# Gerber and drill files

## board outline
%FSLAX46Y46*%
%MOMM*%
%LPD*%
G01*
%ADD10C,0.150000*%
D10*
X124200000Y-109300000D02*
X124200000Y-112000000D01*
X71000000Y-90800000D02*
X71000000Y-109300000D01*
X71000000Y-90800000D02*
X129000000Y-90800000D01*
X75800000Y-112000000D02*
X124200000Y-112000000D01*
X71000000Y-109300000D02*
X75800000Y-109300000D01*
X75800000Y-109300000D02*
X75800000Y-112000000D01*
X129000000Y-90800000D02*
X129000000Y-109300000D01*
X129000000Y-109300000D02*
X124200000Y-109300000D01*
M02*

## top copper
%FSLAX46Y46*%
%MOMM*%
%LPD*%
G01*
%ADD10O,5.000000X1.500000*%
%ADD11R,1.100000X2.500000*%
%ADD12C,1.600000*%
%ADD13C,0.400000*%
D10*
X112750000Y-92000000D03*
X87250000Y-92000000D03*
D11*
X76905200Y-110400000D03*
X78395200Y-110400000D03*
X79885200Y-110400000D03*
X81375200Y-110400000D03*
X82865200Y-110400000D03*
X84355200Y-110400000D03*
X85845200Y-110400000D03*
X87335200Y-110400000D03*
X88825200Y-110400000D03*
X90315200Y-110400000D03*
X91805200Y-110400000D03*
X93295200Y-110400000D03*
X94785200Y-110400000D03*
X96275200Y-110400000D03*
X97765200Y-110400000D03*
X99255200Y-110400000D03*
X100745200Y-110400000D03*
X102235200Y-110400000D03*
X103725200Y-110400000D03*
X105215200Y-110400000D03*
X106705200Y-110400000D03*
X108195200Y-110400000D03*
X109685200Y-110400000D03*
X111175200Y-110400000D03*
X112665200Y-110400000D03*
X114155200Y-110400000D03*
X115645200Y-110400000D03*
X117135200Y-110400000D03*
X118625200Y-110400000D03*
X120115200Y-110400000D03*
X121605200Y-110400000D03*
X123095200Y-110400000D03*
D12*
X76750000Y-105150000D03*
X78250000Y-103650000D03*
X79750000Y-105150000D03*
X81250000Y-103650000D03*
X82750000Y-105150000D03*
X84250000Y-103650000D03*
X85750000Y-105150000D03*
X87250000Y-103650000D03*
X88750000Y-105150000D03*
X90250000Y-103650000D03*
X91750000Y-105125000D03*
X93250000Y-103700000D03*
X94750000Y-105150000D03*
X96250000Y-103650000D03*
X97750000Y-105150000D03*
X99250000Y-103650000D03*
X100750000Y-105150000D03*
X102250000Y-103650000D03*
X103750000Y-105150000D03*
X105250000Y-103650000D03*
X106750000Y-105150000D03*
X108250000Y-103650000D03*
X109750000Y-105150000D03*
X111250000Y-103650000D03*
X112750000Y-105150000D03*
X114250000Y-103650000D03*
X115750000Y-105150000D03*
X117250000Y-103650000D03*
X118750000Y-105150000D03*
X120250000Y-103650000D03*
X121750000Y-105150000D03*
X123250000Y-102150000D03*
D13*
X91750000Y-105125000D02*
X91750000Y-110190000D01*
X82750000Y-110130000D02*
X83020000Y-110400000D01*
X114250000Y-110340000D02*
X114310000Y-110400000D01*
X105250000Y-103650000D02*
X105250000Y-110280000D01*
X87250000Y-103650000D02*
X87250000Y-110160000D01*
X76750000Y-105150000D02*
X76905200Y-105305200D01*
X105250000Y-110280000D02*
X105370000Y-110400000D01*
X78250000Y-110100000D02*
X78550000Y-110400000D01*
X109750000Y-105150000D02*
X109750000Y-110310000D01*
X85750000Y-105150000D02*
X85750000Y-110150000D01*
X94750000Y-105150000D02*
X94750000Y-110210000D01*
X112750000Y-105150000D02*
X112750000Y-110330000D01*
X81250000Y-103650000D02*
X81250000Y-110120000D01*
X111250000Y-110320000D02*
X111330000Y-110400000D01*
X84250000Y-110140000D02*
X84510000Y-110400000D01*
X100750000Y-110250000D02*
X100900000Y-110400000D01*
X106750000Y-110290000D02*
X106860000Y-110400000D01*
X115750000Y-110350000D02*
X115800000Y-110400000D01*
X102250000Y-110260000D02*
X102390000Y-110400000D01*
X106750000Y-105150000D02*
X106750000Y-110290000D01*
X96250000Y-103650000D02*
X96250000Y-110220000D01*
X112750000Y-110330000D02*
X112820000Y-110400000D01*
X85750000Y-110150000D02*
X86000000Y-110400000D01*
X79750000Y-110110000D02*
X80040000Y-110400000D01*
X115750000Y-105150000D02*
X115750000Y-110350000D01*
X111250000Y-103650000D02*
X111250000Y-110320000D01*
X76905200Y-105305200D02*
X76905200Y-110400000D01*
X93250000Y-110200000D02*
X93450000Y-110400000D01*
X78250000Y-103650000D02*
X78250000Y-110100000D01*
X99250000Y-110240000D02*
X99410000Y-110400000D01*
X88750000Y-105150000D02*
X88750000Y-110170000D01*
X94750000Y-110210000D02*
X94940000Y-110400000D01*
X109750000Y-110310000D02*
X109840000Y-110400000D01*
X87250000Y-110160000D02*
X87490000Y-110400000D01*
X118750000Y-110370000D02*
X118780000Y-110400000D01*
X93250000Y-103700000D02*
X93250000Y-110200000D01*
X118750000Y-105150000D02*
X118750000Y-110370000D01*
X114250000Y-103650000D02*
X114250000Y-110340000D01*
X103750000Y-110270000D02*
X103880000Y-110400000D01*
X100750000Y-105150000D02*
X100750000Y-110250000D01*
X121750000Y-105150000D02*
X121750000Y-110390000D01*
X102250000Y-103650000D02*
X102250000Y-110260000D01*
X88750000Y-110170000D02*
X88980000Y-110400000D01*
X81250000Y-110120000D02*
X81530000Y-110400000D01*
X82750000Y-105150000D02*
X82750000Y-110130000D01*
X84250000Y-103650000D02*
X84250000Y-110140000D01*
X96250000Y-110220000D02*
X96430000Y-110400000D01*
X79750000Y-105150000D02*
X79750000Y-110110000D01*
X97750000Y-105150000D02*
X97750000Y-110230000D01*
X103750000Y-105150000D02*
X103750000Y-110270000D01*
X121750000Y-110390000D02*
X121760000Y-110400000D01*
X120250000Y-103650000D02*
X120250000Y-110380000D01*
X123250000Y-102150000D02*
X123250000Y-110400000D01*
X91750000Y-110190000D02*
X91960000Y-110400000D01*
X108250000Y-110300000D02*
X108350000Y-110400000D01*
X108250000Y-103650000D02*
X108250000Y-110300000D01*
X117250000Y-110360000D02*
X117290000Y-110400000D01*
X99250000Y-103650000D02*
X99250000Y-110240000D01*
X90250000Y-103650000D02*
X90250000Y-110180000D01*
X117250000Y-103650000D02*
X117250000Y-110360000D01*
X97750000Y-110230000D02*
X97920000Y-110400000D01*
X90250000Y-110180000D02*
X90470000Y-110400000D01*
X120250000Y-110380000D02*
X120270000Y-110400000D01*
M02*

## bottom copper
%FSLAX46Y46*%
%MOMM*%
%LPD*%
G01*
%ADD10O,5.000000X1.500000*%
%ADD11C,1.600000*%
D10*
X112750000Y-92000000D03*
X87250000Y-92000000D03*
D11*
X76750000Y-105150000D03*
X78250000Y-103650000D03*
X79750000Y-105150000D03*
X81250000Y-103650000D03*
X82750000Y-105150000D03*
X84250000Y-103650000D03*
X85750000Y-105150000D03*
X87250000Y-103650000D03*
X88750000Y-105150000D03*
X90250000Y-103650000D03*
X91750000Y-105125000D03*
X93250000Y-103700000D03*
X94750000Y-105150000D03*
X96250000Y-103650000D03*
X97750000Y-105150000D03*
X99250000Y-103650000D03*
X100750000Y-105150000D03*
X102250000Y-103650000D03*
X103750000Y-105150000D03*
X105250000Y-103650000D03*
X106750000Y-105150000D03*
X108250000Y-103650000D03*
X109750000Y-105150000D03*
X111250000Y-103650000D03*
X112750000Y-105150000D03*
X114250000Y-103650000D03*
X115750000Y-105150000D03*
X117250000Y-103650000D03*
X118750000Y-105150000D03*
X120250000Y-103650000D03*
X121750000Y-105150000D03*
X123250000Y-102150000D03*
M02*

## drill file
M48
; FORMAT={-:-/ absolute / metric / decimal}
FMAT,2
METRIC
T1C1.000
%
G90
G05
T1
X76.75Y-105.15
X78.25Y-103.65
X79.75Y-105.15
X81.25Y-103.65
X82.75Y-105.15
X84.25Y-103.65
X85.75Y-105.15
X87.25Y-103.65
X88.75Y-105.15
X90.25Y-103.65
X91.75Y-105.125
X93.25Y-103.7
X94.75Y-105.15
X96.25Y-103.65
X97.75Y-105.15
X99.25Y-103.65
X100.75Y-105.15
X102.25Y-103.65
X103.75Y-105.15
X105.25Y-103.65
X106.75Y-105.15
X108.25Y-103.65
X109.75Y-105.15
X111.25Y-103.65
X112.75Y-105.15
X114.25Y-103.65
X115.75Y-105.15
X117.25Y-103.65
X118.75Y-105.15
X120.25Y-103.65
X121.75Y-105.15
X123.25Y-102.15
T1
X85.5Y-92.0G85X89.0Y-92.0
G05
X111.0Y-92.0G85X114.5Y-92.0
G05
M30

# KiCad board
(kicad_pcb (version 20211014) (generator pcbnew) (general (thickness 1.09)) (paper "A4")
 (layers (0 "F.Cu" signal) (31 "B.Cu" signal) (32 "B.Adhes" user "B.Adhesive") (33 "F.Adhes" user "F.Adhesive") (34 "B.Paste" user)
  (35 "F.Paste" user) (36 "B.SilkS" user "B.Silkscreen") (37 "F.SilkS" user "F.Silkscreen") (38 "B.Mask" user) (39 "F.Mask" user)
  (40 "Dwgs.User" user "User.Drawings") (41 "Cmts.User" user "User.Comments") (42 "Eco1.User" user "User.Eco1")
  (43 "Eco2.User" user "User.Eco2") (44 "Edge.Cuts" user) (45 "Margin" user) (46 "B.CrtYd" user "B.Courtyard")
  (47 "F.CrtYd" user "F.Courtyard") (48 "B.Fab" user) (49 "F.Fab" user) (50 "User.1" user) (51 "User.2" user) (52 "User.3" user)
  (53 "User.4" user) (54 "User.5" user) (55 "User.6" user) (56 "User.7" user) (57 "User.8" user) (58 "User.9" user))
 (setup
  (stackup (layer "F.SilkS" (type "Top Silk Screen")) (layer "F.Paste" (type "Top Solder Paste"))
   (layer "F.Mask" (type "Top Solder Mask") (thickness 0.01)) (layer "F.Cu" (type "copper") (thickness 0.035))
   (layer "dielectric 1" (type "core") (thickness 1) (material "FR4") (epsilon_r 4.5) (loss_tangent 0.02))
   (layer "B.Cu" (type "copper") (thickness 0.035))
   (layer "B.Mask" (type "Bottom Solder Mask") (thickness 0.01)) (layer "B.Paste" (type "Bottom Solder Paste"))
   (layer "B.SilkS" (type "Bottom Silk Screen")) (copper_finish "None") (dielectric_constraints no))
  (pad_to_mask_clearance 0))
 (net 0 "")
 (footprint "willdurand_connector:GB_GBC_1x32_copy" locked (layer "F.Cu") (at 100 100)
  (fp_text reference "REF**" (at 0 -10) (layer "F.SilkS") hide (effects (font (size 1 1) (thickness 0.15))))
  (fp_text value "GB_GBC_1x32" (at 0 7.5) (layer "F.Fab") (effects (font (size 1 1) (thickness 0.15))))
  (pad "" thru_hole oval locked (at 12.75 -8) (size 5 1.5) (drill oval 4.5 1) (layers *.Cu *.Mask))
  (pad "" thru_hole oval locked (at -12.75 -8) (size 5 1.5) (drill oval 4.5 1) (layers *.Cu *.Mask))
  (pad "1" connect rect locked (at -23.0948 10.4) (size 1.1 2.5) (layers "F.Cu" "F.Mask"))
  (pad "2" connect rect locked (at -21.6048 10.4) (size 1.1 2.5) (layers "F.Cu" "F.Mask"))
  (pad "3" connect rect locked (at -20.1148 10.4) (size 1.1 2.5) (layers "F.Cu" "F.Mask"))
  (pad "4" connect rect locked (at -18.6248 10.4) (size 1.1 2.5) (layers "F.Cu" "F.Mask"))
  (pad "5" connect rect locked (at -17.1348 10.4) (size 1.1 2.5) (layers "F.Cu" "F.Mask"))
  (pad "6" connect rect locked (at -15.6448 10.4) (size 1.1 2.5) (layers "F.Cu" "F.Mask"))
  (pad "7" connect rect locked (at -14.1548 10.4) (size 1.1 2.5) (layers "F.Cu" "F.Mask"))
  (pad "8" connect rect locked (at -12.6648 10.4) (size 1.1 2.5) (layers "F.Cu" "F.Mask"))
  (pad "9" connect rect locked (at -11.1748 10.4) (size 1.1 2.5) (layers "F.Cu" "F.Mask"))
  (pad "10" connect rect locked (at -9.6848 10.4) (size 1.1 2.5) (layers "F.Cu" "F.Mask"))
  (pad "11" connect rect locked (at -8.1948 10.4) (size 1.1 2.5) (layers "F.Cu" "F.Mask"))
  (pad "12" connect rect locked (at -6.7048 10.4) (size 1.1 2.5) (layers "F.Cu" "F.Mask"))
  (pad "13" connect rect locked (at -5.2148 10.4) (size 1.1 2.5) (layers "F.Cu" "F.Mask"))
  (pad "14" connect rect locked (at -3.7248 10.4) (size 1.1 2.5) (layers "F.Cu" "F.Mask"))
  (pad "15" connect rect locked (at -2.2348 10.4) (size 1.1 2.5) (layers "F.Cu" "F.Mask"))
  (pad "16" connect rect locked (at -0.7448 10.4) (size 1.1 2.5) (layers "F.Cu" "F.Mask"))
  (pad "17" connect rect locked (at 0.7452 10.4) (size 1.1 2.5) (layers "F.Cu" "F.Mask"))
  (pad "18" connect rect locked (at 2.2352 10.4) (size 1.1 2.5) (layers "F.Cu" "F.Mask"))
  (pad "19" connect rect locked (at 3.7252 10.4) (size 1.1 2.5) (layers "F.Cu" "F.Mask"))
  (pad "20" connect rect locked (at 5.2152 10.4) (size 1.1 2.5) (layers "F.Cu" "F.Mask"))
  (pad "21" connect rect locked (at 6.7052 10.4) (size 1.1 2.5) (layers "F.Cu" "F.Mask"))
  (pad "22" connect rect locked (at 8.1952 10.4) (size 1.1 2.5) (layers "F.Cu" "F.Mask"))
  (pad "23" connect rect locked (at 9.6852 10.4) (size 1.1 2.5) (layers "F.Cu" "F.Mask"))
  (pad "24" connect rect locked (at 11.1752 10.4) (size 1.1 2.5) (layers "F.Cu" "F.Mask"))
  (pad "25" connect rect locked (at 12.6652 10.4) (size 1.1 2.5) (layers "F.Cu" "F.Mask"))
  (pad "26" connect rect locked (at 14.1552 10.4) (size 1.1 2.5) (layers "F.Cu" "F.Mask"))
  (pad "27" connect rect locked (at 15.6452 10.4) (size 1.1 2.5) (layers "F.Cu" "F.Mask"))
  (pad "28" connect rect locked (at 17.1352 10.4) (size 1.1 2.5) (layers "F.Cu" "F.Mask"))
  (pad "29" connect rect locked (at 18.6252 10.4) (size 1.1 2.5) (layers "F.Cu" "F.Mask"))
  (pad "30" connect rect locked (at 20.1152 10.4) (size 1.1 2.5) (layers "F.Cu" "F.Mask"))
  (pad "31" connect rect locked (at 21.6052 10.4) (size 1.1 2.5) (layers "F.Cu" "F.Mask"))
  (pad "32" connect rect locked (at 23.0952 10.4) (size 1.1 2.5) (layers "F.Cu" "F.Mask")))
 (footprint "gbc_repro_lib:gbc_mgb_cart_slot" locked (layer "B.Cu") (at 100 105.15 180)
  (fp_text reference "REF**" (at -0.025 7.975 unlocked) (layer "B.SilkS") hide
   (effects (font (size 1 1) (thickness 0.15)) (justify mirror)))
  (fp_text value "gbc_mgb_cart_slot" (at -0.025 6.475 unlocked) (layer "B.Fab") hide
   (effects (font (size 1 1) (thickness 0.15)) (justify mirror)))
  (pad "1" thru_hole circle locked (at 23.25 0 180) (size 1.6 1.6) (drill 1) (layers *.Cu *.Mask))
  (pad "2" thru_hole circle locked (at 21.75 1.5 180) (size 1.6 1.6) (drill 1) (layers *.Cu *.Mask))
  (pad "3" thru_hole circle locked (at 20.25 0 180) (size 1.6 1.6) (drill 1) (layers *.Cu *.Mask))
  (pad "4" thru_hole circle locked (at 18.75 1.5 180) (size 1.6 1.6) (drill 1) (layers *.Cu *.Mask))
  (pad "5" thru_hole circle locked (at 17.25 0 180) (size 1.6 1.6) (drill 1) (layers *.Cu *.Mask))
  (pad "6" thru_hole circle locked (at 15.75 1.5 180) (size 1.6 1.6) (drill 1) (layers *.Cu *.Mask))
  (pad "7" thru_hole circle locked (at 14.25 0 180) (size 1.6 1.6) (drill 1) (layers *.Cu *.Mask))
  (pad "8" thru_hole circle locked (at 12.75 1.5 180) (size 1.6 1.6) (drill 1) (layers *.Cu *.Mask))
  (pad "9" thru_hole circle locked (at 11.25 0 180) (size 1.6 1.6) (drill 1) (layers *.Cu *.Mask))
  (pad "10" thru_hole circle locked (at 9.75 1.5 180) (size 1.6 1.6) (drill 1) (layers *.Cu *.Mask))
  (pad "11" thru_hole circle locked (at 8.25 0.025 180) (size 1.6 1.6) (drill 1) (layers *.Cu *.Mask))
  (pad "12" thru_hole circle locked (at 6.75 1.45 180) (size 1.6 1.6) (drill 1) (layers *.Cu *.Mask))
  (pad "13" thru_hole circle locked (at 5.25 0 180) (size 1.6 1.6) (drill 1) (layers *.Cu *.Mask))
  (pad "14" thru_hole circle locked (at 3.75 1.5 180) (size 1.6 1.6) (drill 1) (layers *.Cu *.Mask))
  (pad "15" thru_hole circle locked (at 2.25 0 180) (size 1.6 1.6) (drill 1) (layers *.Cu *.Mask))
  (pad "16" thru_hole circle locked (at 0.75 1.5 180) (size 1.6 1.6) (drill 1) (layers *.Cu *.Mask))
  (pad "17" thru_hole circle locked (at -0.75 0 180) (size 1.6 1.6) (drill 1) (layers *.Cu *.Mask))
  (pad "18" thru_hole circle locked (at -2.25 1.5 180) (size 1.6 1.6) (drill 1) (layers *.Cu *.Mask))
  (pad "19" thru_hole circle locked (at -3.75 0 180) (size 1.6 1.6) (drill 1) (layers *.Cu *.Mask))
  (pad "20" thru_hole circle locked (at -5.25 1.5 180) (size 1.6 1.6) (drill 1) (layers *.Cu *.Mask))
  (pad "21" thru_hole circle locked (at -6.75 0 180) (size 1.6 1.6) (drill 1) (layers *.Cu *.Mask))
  (pad "22" thru_hole circle locked (at -8.25 1.5 180) (size 1.6 1.6) (drill 1) (layers *.Cu *.Mask))
  (pad "23" thru_hole circle locked (at -9.75 0 180) (size 1.6 1.6) (drill 1) (layers *.Cu *.Mask))
  (pad "24" thru_hole circle locked (at -11.25 1.5 180) (size 1.6 1.6) (drill 1) (layers *.Cu *.Mask))
  (pad "25" thru_hole circle locked (at -12.75 0 180) (size 1.6 1.6) (drill 1) (layers *.Cu *.Mask))
  (pad "26" thru_hole circle locked (at -14.25 1.5 180) (size 1.6 1.6) (drill 1) (layers *.Cu *.Mask))
  (pad "27" thru_hole circle locked (at -15.75 0 180) (size 1.6 1.6) (drill 1) (layers *.Cu *.Mask))
  (pad "28" thru_hole circle locked (at -17.25 1.5 180) (size 1.6 1.6) (drill 1) (layers *.Cu *.Mask))
  (pad "29" thru_hole circle locked (at -18.75 0 180) (size 1.6 1.6) (drill 1) (layers *.Cu *.Mask))
  (pad "30" thru_hole circle locked (at -20.25 1.5 180) (size 1.6 1.6) (drill 1) (layers *.Cu *.Mask))
  (pad "31" thru_hole circle locked (at -21.75 0 180) (size 1.6 1.6) (drill 1) (layers *.Cu *.Mask))
  (pad "32" thru_hole circle locked (at -23.25 3 180) (size 1.6 1.6) (drill 1) (layers *.Cu *.Mask)))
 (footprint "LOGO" (layer "B.Cu") (at 97.005907 108.575795 180)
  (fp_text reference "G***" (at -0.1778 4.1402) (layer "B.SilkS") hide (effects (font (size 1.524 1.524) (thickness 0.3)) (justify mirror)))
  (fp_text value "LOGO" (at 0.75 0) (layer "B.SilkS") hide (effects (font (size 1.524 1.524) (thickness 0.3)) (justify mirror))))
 (gr_line (start 124.2 109.3) (end 124.2 112) (layer "Edge.Cuts") (width 0.15))
 (gr_line (start 71 90.8) (end 71 109.3) (layer "Edge.Cuts") (width 0.15))
 (gr_line (start 71 90.8) (end 129 90.8) (layer "Edge.Cuts") (width 0.15))
 (gr_line (start 75.8 112) (end 124.2 112) (layer "Edge.Cuts") (width 0.15))
 (gr_line (start 71 109.3) (end 75.8 109.3) (layer "Edge.Cuts") (width 0.15))
 (gr_line (start 75.8 109.3) (end 75.8 112) (layer "Edge.Cuts") (width 0.15))
 (gr_line (start 129 90.8) (end 129 109.3) (layer "Edge.Cuts") (width 0.15))
 (gr_line (start 129 109.3) (end 124.2 109.3) (layer "Edge.Cuts") (width 0.15))
 (segment (start 91.75 105.125) (end 91.75 110.19) (width 0.4) (layer "F.Cu") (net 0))
 (segment (start 82.75 110.13) (end 83.02 110.4) (width 0.4) (layer "F.Cu") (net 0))
 (segment (start 114.25 110.34) (end 114.31 110.4) (width 0.4) (layer "F.Cu") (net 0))
 (segment (start 105.25 103.65) (end 105.25 110.28) (width 0.4) (layer "F.Cu") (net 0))
 (segment (start 87.25 103.65) (end 87.25 110.16) (width 0.4) (layer "F.Cu") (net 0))
 (segment (start 76.75 105.15) (end 76.9052 105.3052) (width 0.4) (layer "F.Cu") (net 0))
 (segment (start 105.25 110.28) (end 105.37 110.4) (width 0.4) (layer "F.Cu") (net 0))
 (segment (start 78.25 110.1) (end 78.55 110.4) (width 0.4) (layer "F.Cu") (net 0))
 (segment (start 109.75 105.15) (end 109.75 110.31) (width 0.4) (layer "F.Cu") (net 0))
 (segment (start 85.75 105.15) (end 85.75 110.15) (width 0.4) (layer "F.Cu") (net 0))
 (segment (start 94.75 105.15) (end 94.75 110.21) (width 0.4) (layer "F.Cu") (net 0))
 (segment (start 112.75 105.15) (end 112.75 110.33) (width 0.4) (layer "F.Cu") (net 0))
 (segment (start 81.25 103.65) (end 81.25 110.12) (width 0.4) (layer "F.Cu") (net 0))
 (segment (start 111.25 110.32) (end 111.33 110.4) (width 0.4) (layer "F.Cu") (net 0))
 (segment (start 84.25 110.14) (end 84.51 110.4) (width 0.4) (layer "F.Cu") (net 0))
 (segment (start 100.75 110.25) (end 100.9 110.4) (width 0.4) (layer "F.Cu") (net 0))
 (segment (start 106.75 110.29) (end 106.86 110.4) (width 0.4) (layer "F.Cu") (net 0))
 (segment (start 115.75 110.35) (end 115.8 110.4) (width 0.4) (layer "F.Cu") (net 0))
 (segment (start 102.25 110.26) (end 102.39 110.4) (width 0.4) (layer "F.Cu") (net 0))
 (segment (start 106.75 105.15) (end 106.75 110.29) (width 0.4) (layer "F.Cu") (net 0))
 (segment (start 96.25 103.65) (end 96.25 110.22) (width 0.4) (layer "F.Cu") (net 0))
 (segment (start 112.75 110.33) (end 112.82 110.4) (width 0.4) (layer "F.Cu") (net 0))
 (segment (start 85.75 110.15) (end 86 110.4) (width 0.4) (layer "F.Cu") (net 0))
 (segment (start 79.75 110.11) (end 80.04 110.4) (width 0.4) (layer "F.Cu") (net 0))
 (segment (start 115.75 105.15) (end 115.75 110.35) (width 0.4) (layer "F.Cu") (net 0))
 (segment (start 111.25 103.65) (end 111.25 110.32) (width 0.4) (layer "F.Cu") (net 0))
 (segment (start 76.9052 105.3052) (end 76.9052 110.4) (width 0.4) (layer "F.Cu") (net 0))
 (segment (start 93.25 110.2) (end 93.45 110.4) (width 0.4) (layer "F.Cu") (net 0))
 (segment (start 78.25 103.65) (end 78.25 110.1) (width 0.4) (layer "F.Cu") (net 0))
 (segment (start 99.25 110.24) (end 99.41 110.4) (width 0.4) (layer "F.Cu") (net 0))
 (segment (start 88.75 105.15) (end 88.75 110.17) (width 0.4) (layer "F.Cu") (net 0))
 (segment (start 94.75 110.21) (end 94.94 110.4) (width 0.4) (layer "F.Cu") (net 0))
 (segment (start 109.75 110.31) (end 109.84 110.4) (width 0.4) (layer "F.Cu") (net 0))
 (segment (start 87.25 110.16) (end 87.49 110.4) (width 0.4) (layer "F.Cu") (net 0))
 (segment (start 118.75 110.37) (end 118.78 110.4) (width 0.4) (layer "F.Cu") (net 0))
 (segment (start 93.25 103.7) (end 93.25 110.2) (width 0.4) (layer "F.Cu") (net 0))
 (segment (start 118.75 105.15) (end 118.75 110.37) (width 0.4) (layer "F.Cu") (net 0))
 (segment (start 114.25 103.65) (end 114.25 110.34) (width 0.4) (layer "F.Cu") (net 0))
 (segment (start 103.75 110.27) (end 103.88 110.4) (width 0.4) (layer "F.Cu") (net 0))
 (segment (start 100.75 105.15) (end 100.75 110.25) (width 0.4) (layer "F.Cu") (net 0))
 (segment (start 121.75 105.15) (end 121.75 110.39) (width 0.4) (layer "F.Cu") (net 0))
 (segment (start 102.25 103.65) (end 102.25 110.26) (width 0.4) (layer "F.Cu") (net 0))
 (segment (start 88.75 110.17) (end 88.98 110.4) (width 0.4) (layer "F.Cu") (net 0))
 (segment (start 81.25 110.12) (end 81.53 110.4) (width 0.4) (layer "F.Cu") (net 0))
 (segment (start 82.75 105.15) (end 82.75 110.13) (width 0.4) (layer "F.Cu") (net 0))
 (segment (start 84.25 103.65) (end 84.25 110.14) (width 0.4) (layer "F.Cu") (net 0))
 (segment (start 96.25 110.22) (end 96.43 110.4) (width 0.4) (layer "F.Cu") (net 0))
 (segment (start 79.75 105.15) (end 79.75 110.11) (width 0.4) (layer "F.Cu") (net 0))
 (segment (start 97.75 105.15) (end 97.75 110.23) (width 0.4) (layer "F.Cu") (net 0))
 (segment (start 103.75 105.15) (end 103.75 110.27) (width 0.4) (layer "F.Cu") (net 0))
 (segment (start 121.75 110.39) (end 121.76 110.4) (width 0.4) (layer "F.Cu") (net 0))
 (segment (start 120.25 103.65) (end 120.25 110.38) (width 0.4) (layer "F.Cu") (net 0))
 (segment (start 123.25 102.15) (end 123.25 110.4) (width 0.4) (layer "F.Cu") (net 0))
 (segment (start 91.75 110.19) (end 91.96 110.4) (width 0.4) (layer "F.Cu") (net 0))
 (segment (start 108.25 110.3) (end 108.35 110.4) (width 0.4) (layer "F.Cu") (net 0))
 (segment (start 108.25 103.65) (end 108.25 110.3) (width 0.4) (layer "F.Cu") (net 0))
 (segment (start 117.25 110.36) (end 117.29 110.4) (width 0.4) (layer "F.Cu") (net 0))
 (segment (start 99.25 103.65) (end 99.25 110.24) (width 0.4) (layer "F.Cu") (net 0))
 (segment (start 90.25 103.65) (end 90.25 110.18) (width 0.4) (layer "F.Cu") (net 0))
 (segment (start 117.25 103.65) (end 117.25 110.36) (width 0.4) (layer "F.Cu") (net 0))
 (segment (start 97.75 110.23) (end 97.92 110.4) (width 0.4) (layer "F.Cu") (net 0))
 (segment (start 90.25 110.18) (end 90.47 110.4) (width 0.4) (layer "F.Cu") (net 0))
 (segment (start 120.25 110.38) (end 120.27 110.4) (width 0.4) (layer "F.Cu") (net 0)))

